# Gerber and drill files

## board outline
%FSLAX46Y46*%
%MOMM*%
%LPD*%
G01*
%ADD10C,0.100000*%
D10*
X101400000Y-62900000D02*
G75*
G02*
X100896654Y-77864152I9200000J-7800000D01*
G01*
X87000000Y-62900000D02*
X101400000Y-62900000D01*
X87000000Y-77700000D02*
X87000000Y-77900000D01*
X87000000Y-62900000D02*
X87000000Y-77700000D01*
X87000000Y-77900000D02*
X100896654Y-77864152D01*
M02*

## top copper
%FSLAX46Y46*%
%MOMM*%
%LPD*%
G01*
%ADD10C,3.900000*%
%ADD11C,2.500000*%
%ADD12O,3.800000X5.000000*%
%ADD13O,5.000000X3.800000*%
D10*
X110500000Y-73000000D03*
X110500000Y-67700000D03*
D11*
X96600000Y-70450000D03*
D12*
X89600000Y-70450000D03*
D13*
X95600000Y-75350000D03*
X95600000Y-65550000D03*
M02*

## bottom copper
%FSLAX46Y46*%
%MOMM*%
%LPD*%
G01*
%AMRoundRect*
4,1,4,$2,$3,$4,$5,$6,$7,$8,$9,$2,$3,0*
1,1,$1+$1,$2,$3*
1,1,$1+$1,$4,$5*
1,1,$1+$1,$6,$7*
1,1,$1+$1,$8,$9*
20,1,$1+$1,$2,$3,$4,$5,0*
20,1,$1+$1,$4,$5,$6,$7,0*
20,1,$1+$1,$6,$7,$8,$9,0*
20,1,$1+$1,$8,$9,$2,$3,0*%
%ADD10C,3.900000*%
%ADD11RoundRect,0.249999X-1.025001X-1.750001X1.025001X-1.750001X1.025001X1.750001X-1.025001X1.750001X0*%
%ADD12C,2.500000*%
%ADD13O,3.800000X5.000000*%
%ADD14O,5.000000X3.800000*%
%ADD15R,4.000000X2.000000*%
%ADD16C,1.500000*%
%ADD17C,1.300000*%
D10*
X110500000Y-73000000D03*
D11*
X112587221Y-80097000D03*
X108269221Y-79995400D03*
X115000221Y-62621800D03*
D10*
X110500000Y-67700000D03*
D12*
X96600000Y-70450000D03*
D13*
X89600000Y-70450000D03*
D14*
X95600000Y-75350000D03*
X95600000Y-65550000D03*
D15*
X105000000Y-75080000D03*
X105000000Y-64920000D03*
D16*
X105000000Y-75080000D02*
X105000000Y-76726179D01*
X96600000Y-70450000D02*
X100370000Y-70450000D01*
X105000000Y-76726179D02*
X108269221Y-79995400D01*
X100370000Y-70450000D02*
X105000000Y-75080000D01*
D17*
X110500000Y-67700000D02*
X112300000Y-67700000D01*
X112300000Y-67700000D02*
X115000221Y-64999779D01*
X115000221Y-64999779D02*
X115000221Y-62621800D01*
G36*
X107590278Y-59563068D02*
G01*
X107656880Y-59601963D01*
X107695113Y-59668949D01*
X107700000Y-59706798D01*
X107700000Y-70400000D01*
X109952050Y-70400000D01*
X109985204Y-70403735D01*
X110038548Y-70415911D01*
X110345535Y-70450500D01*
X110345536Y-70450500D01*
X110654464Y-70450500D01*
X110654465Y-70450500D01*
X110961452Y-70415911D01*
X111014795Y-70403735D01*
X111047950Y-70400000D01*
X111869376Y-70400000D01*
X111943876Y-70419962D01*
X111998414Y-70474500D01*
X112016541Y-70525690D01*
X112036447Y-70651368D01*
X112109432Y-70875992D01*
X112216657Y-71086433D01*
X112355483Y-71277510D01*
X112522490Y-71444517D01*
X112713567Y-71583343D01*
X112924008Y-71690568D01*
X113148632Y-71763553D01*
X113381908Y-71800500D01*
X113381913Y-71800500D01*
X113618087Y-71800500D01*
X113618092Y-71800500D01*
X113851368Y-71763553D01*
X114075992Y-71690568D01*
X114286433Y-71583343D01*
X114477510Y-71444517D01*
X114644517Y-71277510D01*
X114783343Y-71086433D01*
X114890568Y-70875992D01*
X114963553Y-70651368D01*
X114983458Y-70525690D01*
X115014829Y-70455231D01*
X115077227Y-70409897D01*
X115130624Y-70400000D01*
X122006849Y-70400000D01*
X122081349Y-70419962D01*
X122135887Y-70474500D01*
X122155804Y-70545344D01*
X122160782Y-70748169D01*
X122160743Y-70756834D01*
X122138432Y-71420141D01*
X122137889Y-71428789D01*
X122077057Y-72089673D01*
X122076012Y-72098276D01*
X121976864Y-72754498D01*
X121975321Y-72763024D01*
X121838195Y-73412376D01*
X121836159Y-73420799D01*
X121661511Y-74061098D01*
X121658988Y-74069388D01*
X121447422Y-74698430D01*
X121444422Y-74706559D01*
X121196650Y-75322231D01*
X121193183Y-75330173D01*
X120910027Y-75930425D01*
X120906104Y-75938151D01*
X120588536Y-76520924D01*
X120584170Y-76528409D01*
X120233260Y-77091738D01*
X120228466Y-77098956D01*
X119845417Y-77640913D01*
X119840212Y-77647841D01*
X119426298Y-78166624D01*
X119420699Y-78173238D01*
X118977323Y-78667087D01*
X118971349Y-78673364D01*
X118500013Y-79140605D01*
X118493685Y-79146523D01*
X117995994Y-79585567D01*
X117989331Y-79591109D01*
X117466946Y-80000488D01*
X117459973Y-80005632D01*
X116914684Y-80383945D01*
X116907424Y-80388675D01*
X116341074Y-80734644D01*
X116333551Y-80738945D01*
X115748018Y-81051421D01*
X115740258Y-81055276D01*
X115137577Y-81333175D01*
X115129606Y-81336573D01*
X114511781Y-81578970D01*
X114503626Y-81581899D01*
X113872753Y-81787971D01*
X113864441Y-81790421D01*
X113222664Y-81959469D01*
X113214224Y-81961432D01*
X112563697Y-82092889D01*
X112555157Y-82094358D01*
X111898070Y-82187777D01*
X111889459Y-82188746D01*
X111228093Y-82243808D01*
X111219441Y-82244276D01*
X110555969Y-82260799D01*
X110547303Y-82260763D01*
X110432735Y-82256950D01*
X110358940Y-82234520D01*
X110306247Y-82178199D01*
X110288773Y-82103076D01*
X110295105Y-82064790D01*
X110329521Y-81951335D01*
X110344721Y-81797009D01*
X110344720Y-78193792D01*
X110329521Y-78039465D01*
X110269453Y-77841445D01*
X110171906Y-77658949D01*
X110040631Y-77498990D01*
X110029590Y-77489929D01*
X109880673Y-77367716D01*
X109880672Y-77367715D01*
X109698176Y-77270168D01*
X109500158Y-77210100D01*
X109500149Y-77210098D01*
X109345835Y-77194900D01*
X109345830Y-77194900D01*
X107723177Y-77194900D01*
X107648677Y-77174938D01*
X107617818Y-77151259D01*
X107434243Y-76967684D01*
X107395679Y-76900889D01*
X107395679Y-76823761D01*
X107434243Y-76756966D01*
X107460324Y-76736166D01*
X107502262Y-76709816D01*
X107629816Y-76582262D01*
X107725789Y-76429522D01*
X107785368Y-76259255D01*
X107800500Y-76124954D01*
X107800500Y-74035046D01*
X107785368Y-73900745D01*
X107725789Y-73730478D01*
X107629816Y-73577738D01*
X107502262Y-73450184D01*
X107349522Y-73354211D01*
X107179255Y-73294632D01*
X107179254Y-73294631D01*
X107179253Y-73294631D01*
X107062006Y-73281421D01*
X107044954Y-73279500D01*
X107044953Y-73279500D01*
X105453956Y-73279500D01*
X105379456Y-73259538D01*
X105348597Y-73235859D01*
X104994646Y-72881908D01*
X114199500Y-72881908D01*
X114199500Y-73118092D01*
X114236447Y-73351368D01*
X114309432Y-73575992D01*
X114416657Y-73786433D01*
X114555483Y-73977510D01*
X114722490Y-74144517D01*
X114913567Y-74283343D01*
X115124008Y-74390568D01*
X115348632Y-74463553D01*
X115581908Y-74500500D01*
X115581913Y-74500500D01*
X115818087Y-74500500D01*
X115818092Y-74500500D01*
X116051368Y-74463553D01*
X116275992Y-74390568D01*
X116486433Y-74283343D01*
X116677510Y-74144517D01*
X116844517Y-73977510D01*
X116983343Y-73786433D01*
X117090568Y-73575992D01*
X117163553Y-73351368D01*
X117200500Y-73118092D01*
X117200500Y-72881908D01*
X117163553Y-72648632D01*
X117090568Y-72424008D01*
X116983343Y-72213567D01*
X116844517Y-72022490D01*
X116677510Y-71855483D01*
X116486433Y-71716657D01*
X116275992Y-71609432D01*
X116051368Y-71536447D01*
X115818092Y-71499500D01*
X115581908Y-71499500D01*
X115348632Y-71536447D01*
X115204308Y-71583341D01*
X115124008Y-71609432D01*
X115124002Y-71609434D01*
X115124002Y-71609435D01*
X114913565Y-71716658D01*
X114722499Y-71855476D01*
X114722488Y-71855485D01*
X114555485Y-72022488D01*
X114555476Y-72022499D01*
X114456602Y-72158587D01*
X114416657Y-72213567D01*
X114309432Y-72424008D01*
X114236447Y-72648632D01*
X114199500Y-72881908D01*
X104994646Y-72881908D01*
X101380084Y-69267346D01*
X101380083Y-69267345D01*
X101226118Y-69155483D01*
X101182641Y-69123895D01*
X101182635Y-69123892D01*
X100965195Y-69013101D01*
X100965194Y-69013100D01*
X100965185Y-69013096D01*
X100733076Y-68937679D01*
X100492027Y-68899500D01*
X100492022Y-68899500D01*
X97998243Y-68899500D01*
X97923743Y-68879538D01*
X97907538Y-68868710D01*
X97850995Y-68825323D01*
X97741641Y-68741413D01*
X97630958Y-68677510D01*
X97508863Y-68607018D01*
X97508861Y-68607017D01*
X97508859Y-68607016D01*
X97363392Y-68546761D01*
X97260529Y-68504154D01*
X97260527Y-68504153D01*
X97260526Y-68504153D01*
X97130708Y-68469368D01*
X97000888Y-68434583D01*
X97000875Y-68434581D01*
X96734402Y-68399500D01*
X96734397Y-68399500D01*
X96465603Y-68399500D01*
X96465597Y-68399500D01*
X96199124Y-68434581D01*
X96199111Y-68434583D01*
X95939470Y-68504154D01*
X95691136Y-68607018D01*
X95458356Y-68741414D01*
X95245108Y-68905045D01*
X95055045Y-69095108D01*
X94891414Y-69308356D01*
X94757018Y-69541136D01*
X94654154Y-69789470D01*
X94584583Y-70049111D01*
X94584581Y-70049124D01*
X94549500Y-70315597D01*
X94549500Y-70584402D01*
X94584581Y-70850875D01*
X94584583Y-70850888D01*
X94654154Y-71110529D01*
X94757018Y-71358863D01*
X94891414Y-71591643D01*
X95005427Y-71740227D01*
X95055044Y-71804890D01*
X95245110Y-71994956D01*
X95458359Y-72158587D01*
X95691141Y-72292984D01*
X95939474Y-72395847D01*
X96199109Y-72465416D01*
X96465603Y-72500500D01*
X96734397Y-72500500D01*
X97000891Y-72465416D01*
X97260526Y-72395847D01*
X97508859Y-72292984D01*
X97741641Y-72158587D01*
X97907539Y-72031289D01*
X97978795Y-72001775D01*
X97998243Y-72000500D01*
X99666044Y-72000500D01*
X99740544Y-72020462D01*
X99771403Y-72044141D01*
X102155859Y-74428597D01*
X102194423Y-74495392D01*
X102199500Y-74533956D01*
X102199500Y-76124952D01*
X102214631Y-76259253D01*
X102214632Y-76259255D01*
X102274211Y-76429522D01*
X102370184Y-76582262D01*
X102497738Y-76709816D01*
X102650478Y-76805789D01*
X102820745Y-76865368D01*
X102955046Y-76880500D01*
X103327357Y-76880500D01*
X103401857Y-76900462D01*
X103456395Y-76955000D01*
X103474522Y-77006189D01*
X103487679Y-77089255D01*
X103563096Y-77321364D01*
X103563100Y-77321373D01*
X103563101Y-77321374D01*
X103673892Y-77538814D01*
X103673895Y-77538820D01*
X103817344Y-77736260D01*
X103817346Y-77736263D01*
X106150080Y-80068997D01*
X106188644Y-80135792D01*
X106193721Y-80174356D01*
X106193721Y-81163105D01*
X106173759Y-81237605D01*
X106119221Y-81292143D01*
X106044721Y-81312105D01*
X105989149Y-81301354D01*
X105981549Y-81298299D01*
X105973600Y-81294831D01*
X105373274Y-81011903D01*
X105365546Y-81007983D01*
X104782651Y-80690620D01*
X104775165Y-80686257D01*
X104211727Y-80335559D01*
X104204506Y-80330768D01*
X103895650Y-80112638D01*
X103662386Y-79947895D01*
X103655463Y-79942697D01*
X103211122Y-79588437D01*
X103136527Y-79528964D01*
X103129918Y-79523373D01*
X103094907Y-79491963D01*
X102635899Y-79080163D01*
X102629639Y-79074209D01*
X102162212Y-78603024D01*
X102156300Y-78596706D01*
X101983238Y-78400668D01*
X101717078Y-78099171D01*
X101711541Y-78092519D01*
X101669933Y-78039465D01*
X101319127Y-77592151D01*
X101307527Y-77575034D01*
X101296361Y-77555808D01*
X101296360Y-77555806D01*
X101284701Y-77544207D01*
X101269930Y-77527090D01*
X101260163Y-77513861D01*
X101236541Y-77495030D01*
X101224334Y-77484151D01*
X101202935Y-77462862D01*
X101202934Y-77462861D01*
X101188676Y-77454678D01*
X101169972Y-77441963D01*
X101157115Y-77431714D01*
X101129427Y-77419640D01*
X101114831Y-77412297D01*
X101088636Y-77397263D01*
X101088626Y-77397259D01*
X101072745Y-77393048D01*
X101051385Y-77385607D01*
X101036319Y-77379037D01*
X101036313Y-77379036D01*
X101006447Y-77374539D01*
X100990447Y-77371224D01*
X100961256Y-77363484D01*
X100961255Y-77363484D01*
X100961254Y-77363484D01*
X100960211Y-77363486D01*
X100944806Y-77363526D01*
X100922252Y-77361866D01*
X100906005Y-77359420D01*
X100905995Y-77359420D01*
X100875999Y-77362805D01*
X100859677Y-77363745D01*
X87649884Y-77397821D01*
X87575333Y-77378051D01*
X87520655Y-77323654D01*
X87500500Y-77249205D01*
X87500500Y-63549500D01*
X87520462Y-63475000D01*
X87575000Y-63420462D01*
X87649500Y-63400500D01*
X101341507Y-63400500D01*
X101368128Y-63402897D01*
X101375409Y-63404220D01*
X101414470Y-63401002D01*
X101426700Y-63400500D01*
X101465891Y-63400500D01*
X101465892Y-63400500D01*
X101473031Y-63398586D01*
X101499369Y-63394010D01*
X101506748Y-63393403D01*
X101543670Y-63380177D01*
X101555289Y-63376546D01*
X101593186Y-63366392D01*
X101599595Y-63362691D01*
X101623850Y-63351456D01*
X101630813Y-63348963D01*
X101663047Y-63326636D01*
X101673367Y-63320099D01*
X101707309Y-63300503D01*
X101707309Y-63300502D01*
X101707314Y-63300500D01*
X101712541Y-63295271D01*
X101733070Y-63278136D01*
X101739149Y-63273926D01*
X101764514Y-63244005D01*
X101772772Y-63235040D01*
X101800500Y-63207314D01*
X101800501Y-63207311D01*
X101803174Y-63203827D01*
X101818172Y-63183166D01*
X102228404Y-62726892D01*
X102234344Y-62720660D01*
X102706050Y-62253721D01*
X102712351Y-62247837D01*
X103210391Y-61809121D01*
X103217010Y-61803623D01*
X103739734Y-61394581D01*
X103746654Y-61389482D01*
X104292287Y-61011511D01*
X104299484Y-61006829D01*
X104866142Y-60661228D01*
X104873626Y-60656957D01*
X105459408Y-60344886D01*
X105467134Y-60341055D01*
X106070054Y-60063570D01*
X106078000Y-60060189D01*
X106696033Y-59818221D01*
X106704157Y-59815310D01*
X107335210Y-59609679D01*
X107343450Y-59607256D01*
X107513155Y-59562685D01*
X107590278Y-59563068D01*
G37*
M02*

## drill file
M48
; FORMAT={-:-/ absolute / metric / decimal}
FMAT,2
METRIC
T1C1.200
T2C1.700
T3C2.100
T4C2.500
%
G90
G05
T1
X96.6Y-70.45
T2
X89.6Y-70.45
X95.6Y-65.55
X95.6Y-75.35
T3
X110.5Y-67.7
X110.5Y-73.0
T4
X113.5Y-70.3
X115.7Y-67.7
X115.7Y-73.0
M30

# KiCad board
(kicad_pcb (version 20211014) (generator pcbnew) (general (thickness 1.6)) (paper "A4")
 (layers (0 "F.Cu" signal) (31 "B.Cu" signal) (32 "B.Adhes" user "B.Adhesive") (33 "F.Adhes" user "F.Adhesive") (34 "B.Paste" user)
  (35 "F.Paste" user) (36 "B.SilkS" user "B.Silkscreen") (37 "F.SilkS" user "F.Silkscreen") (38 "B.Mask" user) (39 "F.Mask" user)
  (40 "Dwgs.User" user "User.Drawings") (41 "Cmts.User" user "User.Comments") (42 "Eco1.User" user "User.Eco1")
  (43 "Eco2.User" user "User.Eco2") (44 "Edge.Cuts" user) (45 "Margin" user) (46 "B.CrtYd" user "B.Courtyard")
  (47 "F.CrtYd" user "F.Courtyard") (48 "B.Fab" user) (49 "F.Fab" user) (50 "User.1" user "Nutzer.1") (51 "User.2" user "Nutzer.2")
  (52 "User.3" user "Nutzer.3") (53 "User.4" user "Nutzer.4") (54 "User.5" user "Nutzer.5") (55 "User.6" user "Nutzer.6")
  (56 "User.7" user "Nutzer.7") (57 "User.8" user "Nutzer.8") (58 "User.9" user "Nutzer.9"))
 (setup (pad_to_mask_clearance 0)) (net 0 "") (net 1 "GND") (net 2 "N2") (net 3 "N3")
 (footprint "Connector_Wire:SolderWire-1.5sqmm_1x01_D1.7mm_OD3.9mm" (layer "F.Cu") (at 110.5 73)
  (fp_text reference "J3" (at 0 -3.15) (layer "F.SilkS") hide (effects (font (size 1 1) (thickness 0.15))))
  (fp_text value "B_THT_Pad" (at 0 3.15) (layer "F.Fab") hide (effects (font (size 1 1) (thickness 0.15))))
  (pad "1" thru_hole circle (at 0 0) (size 3.9 3.9) (drill 2.1) (layers *.Cu *.Mask) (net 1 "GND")))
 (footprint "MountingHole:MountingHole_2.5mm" (layer "F.Cu") (at 113.5 70.3)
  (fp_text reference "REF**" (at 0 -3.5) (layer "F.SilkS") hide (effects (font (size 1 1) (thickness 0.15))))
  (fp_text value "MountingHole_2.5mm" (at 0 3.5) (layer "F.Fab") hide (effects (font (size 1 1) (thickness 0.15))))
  (pad "" np_thru_hole circle (at 0 0) (size 2.5 2.5) (drill 2.5) (layers *.Cu *.Mask)))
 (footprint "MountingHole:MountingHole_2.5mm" (layer "F.Cu") (at 115.7 73)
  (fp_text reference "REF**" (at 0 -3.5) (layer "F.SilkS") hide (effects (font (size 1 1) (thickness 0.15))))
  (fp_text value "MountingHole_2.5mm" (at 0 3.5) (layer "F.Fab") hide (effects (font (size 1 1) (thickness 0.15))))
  (pad "" np_thru_hole circle (at 0 0) (size 2.5 2.5) (drill 2.5) (layers *.Cu *.Mask)))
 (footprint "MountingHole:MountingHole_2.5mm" (layer "F.Cu") (at 115.7 67.7)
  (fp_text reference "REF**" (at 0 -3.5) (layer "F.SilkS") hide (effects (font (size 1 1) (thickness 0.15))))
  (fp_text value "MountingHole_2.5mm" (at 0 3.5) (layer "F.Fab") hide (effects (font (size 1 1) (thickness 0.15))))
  (pad "" np_thru_hole circle (at 0 0) (size 2.5 2.5) (drill 2.5) (layers *.Cu *.Mask)))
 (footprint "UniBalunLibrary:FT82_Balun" (layer "F.Cu") (at 110.555221 70.7498)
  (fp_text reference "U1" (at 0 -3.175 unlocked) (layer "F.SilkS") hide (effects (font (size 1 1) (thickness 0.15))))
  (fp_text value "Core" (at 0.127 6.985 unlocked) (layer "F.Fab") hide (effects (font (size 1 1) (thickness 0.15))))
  (pad "1" smd roundrect (at 2.032 9.3472) (size 2.55 4) (layers "B.Cu" "B.Paste" "B.Mask") (roundrect_rratio 0.09803882353) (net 1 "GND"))
  (pad "2" smd roundrect (at -2.286 9.2456) (size 2.55 4) (layers "B.Cu" "B.Paste" "B.Mask") (roundrect_rratio 0.09803882353) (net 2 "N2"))
  (pad "3" smd roundrect (at 4.445 -8.128) (size 2.55 4) (layers "B.Cu" "B.Paste" "B.Mask") (roundrect_rratio 0.09803882353) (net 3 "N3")))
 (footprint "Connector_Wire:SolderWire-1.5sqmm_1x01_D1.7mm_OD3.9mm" (layer "F.Cu") (at 110.5 67.7)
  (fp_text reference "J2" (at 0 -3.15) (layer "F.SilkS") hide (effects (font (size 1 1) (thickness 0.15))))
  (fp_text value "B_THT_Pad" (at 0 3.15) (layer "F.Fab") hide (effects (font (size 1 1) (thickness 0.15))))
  (pad "1" thru_hole circle (at 0 0) (size 3.9 3.9) (drill 2.1) (layers *.Cu *.Mask) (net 3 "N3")))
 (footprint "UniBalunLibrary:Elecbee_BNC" (layer "F.Cu") (at 95.6 65.55 -90)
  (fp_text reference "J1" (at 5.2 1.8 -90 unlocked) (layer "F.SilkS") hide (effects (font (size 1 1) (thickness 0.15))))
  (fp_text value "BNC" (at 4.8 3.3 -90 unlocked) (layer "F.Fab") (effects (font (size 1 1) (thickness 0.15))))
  (pad "1" thru_hole circle (at 4.9 -1 270) (size 2.5 2.5) (drill 1.2) (layers *.Cu *.Mask) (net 2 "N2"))
  (pad "2" thru_hole oval (at 4.9 6) (size 3.8 5) (drill 1.7) (layers *.Cu *.Mask) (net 1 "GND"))
  (pad "2" thru_hole oval (at 9.8 0 270) (size 3.8 5) (drill 1.7) (layers *.Cu *.Mask) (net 1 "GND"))
  (pad "2" thru_hole oval (at 0 0 270) (size 3.8 5) (drill 1.7) (layers *.Cu *.Mask) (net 1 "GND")))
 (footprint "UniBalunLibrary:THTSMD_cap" (layer "B.Cu") (at 105 70 90)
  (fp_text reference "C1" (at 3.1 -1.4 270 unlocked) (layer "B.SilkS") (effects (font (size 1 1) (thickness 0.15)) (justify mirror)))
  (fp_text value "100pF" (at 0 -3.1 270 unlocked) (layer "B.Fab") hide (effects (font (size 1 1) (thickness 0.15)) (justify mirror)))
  (pad "1" smd rect (at -5.08 0 90) (size 2 4) (layers "B.Cu" "B.Paste" "B.Mask") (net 2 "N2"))
  (pad "2" smd rect (at 5.08 0 90) (size 2 4) (layers "B.Cu" "B.Paste" "B.Mask") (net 1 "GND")))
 (gr_arc (start 101.4 62.9) (mid 122.654691 71.105481) (end 100.896654 77.864152) (layer "Edge.Cuts") (width 0.1))
 (gr_line (start 87 62.9) (end 101.4 62.9) (layer "Edge.Cuts") (width 0.1))
 (gr_line (start 87 77.7) (end 87 77.9) (layer "Edge.Cuts") (width 0.1))
 (gr_line (start 87 62.9) (end 87 77.7) (layer "Edge.Cuts") (width 0.1))
 (gr_line (start 87 77.9) (end 100.896654 77.864152) (layer "Edge.Cuts") (width 0.1))
 (segment (start 105 75.08) (end 105 76.726179) (width 1.5) (layer "B.Cu") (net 2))
 (segment (start 96.6 70.45) (end 100.37 70.45) (width 1.5) (layer "B.Cu") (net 2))
 (segment (start 105 76.726179) (end 108.269221 79.9954) (width 1.5) (layer "B.Cu") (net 2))
 (segment (start 100.37 70.45) (end 105 75.08) (width 1.5) (layer "B.Cu") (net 2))
 (segment (start 110.5 67.7) (end 112.3 67.7) (width 1.3) (layer "B.Cu") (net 3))
 (segment (start 112.3 67.7) (end 115.000221 64.999779) (width 1.3) (layer "B.Cu") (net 3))
 (segment (start 115.000221 64.999779) (end 115.000221 62.6218) (width 1.3) (layer "B.Cu") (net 3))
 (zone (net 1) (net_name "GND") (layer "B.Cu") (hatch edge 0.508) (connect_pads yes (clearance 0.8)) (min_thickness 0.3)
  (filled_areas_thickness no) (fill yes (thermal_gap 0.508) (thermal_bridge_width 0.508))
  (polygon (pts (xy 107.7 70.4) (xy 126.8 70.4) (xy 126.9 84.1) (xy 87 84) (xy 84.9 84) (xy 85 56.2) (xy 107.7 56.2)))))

